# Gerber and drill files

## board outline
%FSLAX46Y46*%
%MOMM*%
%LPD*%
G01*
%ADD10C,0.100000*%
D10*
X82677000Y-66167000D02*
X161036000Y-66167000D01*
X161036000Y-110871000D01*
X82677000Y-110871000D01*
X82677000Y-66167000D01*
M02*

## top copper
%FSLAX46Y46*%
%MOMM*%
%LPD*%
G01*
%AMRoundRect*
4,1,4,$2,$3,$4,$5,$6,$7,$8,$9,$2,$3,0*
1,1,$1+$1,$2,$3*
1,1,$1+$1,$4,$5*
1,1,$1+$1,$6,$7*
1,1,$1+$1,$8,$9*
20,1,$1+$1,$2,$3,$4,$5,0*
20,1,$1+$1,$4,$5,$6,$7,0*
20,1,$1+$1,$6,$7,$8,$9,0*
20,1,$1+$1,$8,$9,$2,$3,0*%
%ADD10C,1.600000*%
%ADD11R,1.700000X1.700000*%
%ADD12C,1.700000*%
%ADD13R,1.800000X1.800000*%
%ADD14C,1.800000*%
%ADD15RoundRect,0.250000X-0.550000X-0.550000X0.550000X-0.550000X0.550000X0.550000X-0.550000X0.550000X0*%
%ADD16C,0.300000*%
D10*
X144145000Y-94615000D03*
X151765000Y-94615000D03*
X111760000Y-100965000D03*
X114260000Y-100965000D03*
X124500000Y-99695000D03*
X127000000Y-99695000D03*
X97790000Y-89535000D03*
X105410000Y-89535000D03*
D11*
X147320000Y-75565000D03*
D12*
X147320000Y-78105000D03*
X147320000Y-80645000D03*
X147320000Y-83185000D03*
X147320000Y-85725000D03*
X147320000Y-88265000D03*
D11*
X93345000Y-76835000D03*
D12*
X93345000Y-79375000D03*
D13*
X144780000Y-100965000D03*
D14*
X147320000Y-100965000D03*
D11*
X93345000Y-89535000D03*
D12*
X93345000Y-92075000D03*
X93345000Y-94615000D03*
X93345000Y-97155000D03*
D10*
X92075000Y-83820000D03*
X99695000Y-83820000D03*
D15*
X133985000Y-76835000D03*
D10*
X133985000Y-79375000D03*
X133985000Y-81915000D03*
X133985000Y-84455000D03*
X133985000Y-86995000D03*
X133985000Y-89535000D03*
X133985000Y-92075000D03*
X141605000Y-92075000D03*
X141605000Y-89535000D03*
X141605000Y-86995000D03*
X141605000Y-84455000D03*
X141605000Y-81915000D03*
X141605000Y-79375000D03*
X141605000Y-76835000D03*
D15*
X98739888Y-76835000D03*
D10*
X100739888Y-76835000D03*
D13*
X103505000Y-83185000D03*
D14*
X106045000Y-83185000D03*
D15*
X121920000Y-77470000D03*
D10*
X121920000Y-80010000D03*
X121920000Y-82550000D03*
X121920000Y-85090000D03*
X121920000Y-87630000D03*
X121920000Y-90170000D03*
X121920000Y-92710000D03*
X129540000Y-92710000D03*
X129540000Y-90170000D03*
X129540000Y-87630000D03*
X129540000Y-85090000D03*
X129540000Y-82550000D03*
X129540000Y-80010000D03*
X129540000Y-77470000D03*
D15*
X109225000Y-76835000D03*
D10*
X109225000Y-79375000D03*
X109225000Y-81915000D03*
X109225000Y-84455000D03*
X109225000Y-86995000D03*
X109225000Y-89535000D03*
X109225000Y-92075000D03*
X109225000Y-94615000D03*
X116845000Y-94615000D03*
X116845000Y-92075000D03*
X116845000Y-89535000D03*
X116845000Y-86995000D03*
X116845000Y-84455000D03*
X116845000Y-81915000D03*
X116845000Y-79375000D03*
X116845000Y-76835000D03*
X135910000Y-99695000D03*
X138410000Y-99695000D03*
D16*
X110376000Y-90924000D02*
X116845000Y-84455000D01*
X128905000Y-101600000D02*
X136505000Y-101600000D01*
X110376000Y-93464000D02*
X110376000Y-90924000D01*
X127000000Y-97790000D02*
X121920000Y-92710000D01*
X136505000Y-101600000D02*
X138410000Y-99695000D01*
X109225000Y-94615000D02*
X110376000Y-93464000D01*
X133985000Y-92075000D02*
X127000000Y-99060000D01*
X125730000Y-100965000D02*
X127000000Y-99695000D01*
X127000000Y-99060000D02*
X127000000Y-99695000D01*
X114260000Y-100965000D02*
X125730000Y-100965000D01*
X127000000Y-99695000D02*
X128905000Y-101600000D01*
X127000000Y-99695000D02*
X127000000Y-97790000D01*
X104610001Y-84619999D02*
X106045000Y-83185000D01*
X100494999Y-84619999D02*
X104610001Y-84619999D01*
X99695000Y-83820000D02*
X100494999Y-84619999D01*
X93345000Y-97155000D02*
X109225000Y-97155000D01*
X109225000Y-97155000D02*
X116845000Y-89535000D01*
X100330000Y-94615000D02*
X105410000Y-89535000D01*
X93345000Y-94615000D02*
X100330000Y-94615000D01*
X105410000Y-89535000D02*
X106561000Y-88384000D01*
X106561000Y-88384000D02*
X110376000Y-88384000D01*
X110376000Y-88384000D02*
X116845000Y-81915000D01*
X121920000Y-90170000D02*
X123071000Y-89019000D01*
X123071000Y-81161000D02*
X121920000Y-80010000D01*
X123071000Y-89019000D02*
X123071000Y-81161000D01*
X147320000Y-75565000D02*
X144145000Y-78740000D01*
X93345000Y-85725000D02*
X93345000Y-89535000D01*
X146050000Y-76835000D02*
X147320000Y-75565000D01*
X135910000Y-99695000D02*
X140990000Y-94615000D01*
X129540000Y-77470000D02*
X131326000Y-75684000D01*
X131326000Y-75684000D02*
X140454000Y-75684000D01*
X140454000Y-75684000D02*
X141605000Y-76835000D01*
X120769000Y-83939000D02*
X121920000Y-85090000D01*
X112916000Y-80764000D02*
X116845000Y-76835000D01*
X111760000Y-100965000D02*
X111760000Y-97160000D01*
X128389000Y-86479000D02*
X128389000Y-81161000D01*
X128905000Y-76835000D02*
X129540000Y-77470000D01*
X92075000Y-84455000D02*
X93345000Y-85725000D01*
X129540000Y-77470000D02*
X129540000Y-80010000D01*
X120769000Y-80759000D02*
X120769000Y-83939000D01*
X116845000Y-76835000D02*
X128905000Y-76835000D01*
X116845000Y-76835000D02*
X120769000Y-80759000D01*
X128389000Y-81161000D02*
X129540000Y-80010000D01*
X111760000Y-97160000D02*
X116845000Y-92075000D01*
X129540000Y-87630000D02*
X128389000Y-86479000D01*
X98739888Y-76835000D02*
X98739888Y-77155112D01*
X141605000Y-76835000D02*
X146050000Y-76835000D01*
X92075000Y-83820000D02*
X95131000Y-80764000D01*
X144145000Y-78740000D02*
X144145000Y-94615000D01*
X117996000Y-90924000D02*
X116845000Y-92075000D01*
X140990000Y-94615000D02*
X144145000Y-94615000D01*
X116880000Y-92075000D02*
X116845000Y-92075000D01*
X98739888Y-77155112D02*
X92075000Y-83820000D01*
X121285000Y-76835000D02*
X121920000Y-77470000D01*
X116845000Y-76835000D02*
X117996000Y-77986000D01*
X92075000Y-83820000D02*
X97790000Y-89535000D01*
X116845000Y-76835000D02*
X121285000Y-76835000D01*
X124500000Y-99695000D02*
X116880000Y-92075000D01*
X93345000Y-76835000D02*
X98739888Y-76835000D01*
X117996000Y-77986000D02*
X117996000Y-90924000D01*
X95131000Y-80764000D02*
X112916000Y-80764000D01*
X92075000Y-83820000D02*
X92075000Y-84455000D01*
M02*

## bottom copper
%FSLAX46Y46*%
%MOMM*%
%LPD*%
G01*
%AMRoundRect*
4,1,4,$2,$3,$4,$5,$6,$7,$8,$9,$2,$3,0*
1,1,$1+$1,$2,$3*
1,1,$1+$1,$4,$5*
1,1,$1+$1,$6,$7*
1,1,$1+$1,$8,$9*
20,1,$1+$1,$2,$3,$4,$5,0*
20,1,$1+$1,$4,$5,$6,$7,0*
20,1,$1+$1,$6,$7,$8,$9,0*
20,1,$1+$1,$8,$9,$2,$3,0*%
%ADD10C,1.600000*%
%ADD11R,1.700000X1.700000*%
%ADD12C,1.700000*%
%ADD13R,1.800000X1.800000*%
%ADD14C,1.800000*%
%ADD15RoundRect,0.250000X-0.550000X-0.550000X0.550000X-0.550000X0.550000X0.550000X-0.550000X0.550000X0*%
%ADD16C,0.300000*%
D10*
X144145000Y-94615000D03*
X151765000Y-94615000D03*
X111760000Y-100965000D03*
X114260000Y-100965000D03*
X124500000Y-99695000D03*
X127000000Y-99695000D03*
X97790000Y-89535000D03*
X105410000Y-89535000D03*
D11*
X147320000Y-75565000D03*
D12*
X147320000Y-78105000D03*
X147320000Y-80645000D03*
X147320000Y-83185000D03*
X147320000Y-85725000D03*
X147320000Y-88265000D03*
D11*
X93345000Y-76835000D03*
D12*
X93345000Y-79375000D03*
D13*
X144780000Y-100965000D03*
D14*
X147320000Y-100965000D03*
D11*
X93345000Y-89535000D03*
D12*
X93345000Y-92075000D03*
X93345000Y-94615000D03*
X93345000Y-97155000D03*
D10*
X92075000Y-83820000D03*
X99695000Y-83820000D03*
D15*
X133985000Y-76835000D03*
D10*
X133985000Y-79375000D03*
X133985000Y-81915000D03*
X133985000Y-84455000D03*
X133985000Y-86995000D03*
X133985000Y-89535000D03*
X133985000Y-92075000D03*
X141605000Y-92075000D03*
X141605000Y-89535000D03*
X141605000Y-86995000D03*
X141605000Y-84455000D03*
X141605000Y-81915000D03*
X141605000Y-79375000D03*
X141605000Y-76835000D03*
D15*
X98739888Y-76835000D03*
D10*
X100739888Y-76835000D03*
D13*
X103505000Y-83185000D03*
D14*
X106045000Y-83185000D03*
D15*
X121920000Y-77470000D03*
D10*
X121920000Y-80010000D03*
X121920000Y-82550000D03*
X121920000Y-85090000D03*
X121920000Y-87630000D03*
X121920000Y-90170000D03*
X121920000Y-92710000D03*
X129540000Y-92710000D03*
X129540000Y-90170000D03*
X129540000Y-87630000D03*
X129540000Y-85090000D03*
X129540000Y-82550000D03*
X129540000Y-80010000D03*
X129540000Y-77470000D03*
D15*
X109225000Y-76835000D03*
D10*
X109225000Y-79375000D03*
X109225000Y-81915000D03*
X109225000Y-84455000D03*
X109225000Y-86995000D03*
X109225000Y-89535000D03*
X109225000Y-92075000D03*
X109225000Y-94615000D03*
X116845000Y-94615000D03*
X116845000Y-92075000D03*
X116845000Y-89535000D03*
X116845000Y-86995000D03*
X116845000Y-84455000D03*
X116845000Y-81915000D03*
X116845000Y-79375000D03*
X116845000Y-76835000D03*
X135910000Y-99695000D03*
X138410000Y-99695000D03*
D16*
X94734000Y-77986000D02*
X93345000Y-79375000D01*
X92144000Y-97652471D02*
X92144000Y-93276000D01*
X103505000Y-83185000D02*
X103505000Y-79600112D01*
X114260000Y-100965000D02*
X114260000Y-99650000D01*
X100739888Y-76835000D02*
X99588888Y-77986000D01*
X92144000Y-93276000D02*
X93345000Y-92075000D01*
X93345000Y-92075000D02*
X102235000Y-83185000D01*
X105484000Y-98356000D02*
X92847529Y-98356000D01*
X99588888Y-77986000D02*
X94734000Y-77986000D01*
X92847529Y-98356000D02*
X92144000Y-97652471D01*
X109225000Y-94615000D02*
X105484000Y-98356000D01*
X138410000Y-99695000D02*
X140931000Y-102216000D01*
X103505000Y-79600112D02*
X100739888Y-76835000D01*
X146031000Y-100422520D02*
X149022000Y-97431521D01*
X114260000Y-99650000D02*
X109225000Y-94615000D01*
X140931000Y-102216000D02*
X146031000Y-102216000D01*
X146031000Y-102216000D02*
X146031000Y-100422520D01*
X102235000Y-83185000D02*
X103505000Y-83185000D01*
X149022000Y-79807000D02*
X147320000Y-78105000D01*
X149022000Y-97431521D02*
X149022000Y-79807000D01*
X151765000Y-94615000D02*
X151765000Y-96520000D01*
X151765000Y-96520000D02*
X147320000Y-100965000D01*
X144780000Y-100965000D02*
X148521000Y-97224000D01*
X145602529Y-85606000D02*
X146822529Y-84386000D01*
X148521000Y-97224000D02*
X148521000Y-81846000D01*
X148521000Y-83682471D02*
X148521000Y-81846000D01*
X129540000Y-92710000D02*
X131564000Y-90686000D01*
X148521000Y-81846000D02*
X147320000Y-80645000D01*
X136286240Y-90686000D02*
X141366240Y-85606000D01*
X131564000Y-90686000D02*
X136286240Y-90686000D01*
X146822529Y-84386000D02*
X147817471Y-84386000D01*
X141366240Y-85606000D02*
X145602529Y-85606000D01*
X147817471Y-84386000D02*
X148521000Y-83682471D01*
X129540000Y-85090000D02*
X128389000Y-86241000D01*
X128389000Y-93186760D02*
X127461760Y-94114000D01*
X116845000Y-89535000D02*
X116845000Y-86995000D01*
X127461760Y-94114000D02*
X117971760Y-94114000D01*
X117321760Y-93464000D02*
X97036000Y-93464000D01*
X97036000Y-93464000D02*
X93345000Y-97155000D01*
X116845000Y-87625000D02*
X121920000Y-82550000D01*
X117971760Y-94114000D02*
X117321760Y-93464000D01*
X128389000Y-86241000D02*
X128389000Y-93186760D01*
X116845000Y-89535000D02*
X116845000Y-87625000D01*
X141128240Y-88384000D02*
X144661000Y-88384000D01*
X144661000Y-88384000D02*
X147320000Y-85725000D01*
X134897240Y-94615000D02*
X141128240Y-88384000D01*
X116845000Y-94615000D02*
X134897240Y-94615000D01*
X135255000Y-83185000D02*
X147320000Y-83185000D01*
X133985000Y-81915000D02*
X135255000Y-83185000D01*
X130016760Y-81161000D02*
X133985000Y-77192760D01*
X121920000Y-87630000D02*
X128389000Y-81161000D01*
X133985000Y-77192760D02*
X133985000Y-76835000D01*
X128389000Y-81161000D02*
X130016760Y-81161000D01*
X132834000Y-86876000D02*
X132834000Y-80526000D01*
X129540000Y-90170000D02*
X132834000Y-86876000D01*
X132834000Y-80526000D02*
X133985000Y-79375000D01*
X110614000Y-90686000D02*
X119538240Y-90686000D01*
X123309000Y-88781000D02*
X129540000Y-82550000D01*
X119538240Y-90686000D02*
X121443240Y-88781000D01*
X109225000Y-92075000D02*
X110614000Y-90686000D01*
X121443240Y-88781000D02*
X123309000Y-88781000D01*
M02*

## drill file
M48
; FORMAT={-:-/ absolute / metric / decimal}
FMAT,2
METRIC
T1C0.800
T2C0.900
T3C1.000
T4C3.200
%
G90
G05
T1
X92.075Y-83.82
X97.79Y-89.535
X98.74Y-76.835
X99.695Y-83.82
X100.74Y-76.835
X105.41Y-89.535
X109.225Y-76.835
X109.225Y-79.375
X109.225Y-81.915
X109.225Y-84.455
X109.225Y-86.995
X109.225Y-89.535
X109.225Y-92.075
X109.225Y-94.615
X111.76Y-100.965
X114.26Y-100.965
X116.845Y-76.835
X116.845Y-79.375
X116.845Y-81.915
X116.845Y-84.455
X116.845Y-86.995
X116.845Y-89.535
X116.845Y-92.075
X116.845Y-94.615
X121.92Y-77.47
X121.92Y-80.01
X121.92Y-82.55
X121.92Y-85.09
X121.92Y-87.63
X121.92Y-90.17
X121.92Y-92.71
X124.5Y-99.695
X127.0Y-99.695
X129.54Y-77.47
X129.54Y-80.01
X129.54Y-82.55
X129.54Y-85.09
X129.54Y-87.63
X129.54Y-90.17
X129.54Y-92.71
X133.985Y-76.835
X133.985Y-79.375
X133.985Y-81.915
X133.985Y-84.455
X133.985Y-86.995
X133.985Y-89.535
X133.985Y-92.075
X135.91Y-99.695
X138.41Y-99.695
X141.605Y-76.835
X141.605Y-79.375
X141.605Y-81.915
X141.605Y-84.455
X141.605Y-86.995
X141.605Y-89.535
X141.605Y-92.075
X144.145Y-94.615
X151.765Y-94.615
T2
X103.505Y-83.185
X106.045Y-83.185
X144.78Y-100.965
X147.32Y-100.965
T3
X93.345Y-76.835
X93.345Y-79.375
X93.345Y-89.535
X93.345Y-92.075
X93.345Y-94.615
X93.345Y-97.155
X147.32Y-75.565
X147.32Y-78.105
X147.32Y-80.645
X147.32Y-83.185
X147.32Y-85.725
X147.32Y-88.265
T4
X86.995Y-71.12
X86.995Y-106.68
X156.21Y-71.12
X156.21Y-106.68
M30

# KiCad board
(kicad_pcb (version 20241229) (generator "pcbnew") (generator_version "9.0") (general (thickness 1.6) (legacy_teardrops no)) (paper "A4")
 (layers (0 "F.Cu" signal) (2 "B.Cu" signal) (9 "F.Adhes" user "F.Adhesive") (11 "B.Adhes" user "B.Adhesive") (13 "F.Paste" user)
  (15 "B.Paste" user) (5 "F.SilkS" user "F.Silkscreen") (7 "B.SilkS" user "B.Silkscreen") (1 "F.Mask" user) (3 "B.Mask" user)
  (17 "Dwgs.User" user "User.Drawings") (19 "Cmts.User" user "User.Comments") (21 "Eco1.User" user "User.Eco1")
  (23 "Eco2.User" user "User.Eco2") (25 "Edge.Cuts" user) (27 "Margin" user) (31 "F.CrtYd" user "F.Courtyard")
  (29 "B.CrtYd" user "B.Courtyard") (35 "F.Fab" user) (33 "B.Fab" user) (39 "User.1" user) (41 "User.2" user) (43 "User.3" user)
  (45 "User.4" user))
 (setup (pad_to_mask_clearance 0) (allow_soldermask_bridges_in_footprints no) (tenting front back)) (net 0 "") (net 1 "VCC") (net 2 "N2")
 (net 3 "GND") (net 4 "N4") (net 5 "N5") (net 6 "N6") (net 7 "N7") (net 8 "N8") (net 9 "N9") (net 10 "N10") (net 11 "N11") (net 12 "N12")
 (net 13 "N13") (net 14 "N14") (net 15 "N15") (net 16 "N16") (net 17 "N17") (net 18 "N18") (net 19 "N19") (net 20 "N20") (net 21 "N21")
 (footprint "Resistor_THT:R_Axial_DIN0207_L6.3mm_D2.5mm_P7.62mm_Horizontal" (layer "F.Cu") (at 144.145 94.615)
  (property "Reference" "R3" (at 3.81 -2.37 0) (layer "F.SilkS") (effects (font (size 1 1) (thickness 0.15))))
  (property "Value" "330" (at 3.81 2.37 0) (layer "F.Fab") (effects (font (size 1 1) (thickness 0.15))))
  (pad "1" thru_hole circle (at 0 0) (size 1.6 1.6) (drill 0.8) (layers "*.Cu" "*.Mask") (remove_unused_layers no) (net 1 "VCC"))
  (pad "2" thru_hole circle (at 7.62 0) (size 1.6 1.6) (drill 0.8) (layers "*.Cu" "*.Mask") (remove_unused_layers no) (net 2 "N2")))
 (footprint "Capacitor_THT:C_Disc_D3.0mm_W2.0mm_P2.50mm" (layer "F.Cu") (at 111.76 100.965)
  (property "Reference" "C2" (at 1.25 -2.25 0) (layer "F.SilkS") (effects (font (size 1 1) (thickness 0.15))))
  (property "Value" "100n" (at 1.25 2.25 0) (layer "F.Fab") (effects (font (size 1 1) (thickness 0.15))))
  (pad "1" thru_hole circle (at 0 0) (size 1.6 1.6) (drill 0.8) (layers "*.Cu" "*.Mask") (remove_unused_layers no) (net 1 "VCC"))
  (pad "2" thru_hole circle (at 2.5 0) (size 1.6 1.6) (drill 0.8) (layers "*.Cu" "*.Mask") (remove_unused_layers no) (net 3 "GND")))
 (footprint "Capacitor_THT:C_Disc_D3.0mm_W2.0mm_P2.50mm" (layer "F.Cu") (at 124.5 99.695)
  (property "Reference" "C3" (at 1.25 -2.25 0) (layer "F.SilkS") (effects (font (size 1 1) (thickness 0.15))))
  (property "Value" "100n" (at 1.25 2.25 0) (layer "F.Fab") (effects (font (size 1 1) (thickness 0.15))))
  (pad "1" thru_hole circle (at 0 0) (size 1.6 1.6) (drill 0.8) (layers "*.Cu" "*.Mask") (remove_unused_layers no) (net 1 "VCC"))
  (pad "2" thru_hole circle (at 2.5 0) (size 1.6 1.6) (drill 0.8) (layers "*.Cu" "*.Mask") (remove_unused_layers no) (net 3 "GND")))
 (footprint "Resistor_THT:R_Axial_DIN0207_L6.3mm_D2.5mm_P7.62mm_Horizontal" (layer "F.Cu") (at 97.79 89.535)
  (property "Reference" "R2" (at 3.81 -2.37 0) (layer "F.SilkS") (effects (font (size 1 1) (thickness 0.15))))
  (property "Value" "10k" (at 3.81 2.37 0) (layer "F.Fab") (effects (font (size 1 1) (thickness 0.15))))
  (pad "1" thru_hole circle (at 0 0) (size 1.6 1.6) (drill 0.8) (layers "*.Cu" "*.Mask") (remove_unused_layers no) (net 1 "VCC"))
  (pad "2" thru_hole circle (at 7.62 0) (size 1.6 1.6) (drill 0.8) (layers "*.Cu" "*.Mask") (remove_unused_layers no) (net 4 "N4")))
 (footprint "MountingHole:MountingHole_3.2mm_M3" (layer "F.Cu") (at 86.995 71.12)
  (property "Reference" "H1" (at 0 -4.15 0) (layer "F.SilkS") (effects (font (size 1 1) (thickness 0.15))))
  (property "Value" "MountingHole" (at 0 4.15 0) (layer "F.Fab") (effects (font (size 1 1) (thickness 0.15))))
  (pad "" np_thru_hole circle (at 0 0) (size 3.2 3.2) (drill 3.2) (layers "*.Cu" "*.Mask")))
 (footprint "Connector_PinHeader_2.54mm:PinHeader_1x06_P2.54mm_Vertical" (layer "F.Cu") (at 147.32 75.565)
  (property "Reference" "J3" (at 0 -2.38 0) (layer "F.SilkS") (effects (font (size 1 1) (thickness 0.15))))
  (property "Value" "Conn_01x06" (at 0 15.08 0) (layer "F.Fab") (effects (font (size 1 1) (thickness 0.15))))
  (pad "1" thru_hole rect (at 0 0) (size 1.7 1.7) (drill 1) (layers "*.Cu" "*.Mask") (remove_unused_layers no) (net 1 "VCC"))
  (pad "2" thru_hole circle (at 0 2.54) (size 1.7 1.7) (drill 1) (layers "*.Cu" "*.Mask") (remove_unused_layers no) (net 3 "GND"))
  (pad "3" thru_hole circle (at 0 5.08) (size 1.7 1.7) (drill 1) (layers "*.Cu" "*.Mask") (remove_unused_layers no) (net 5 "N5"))
  (pad "4" thru_hole circle (at 0 7.62) (size 1.7 1.7) (drill 1) (layers "*.Cu" "*.Mask") (remove_unused_layers no) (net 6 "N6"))
  (pad "5" thru_hole circle (at 0 10.16) (size 1.7 1.7) (drill 1) (layers "*.Cu" "*.Mask") (remove_unused_layers no) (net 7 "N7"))
  (pad "6" thru_hole circle (at 0 12.7) (size 1.7 1.7) (drill 1) (layers "*.Cu" "*.Mask") (remove_unused_layers no) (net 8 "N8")))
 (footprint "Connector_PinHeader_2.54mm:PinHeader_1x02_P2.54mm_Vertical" (layer "F.Cu") (at 93.345 76.835)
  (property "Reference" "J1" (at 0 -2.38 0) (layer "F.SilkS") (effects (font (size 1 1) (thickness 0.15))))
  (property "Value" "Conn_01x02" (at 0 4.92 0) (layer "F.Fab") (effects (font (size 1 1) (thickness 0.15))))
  (pad "1" thru_hole rect (at 0 0) (size 1.7 1.7) (drill 1) (layers "*.Cu" "*.Mask") (remove_unused_layers no) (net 1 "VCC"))
  (pad "2" thru_hole circle (at 0 2.54) (size 1.7 1.7) (drill 1) (layers "*.Cu" "*.Mask") (remove_unused_layers no) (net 3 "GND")))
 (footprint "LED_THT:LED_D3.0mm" (layer "F.Cu") (at 144.78 100.965)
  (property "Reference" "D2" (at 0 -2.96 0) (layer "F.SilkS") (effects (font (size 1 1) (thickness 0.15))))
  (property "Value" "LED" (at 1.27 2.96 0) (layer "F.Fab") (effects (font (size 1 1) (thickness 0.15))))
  (pad "1" thru_hole rect (at 0 0) (size 1.8 1.8) (drill 0.9) (layers "*.Cu" "*.Mask") (remove_unused_layers no) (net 5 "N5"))
  (pad "2" thru_hole circle (at 2.54 0) (size 1.8 1.8) (drill 0.9) (layers "*.Cu" "*.Mask") (remove_unused_layers no) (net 2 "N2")))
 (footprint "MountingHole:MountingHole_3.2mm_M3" (layer "F.Cu") (at 86.995 106.68)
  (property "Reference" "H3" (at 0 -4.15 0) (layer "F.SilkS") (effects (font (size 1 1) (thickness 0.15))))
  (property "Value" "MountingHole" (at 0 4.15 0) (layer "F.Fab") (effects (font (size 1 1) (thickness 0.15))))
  (pad "" np_thru_hole circle (at 0 0) (size 3.2 3.2) (drill 3.2) (layers "*.Cu" "*.Mask")))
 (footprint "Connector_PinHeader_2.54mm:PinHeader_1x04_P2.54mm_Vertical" (layer "F.Cu") (at 93.345 89.535)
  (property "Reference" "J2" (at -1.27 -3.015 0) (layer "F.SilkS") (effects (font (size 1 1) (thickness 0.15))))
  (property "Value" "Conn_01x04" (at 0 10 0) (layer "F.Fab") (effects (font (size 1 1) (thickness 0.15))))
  (pad "1" thru_hole rect (at 0 0) (size 1.7 1.7) (drill 1) (layers "*.Cu" "*.Mask") (remove_unused_layers no) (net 1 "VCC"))
  (pad "2" thru_hole circle (at 0 2.54) (size 1.7 1.7) (drill 1) (layers "*.Cu" "*.Mask") (remove_unused_layers no) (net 3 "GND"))
  (pad "3" thru_hole circle (at 0 5.08) (size 1.7 1.7) (drill 1) (layers "*.Cu" "*.Mask") (remove_unused_layers no) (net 4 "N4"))
  (pad "4" thru_hole circle (at 0 7.62) (size 1.7 1.7) (drill 1) (layers "*.Cu" "*.Mask") (remove_unused_layers no) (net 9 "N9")))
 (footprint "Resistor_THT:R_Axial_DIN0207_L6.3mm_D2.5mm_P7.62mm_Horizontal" (layer "F.Cu") (at 92.075 83.82)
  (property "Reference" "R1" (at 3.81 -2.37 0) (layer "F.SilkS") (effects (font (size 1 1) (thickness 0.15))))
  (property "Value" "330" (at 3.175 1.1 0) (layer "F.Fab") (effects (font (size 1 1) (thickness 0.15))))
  (pad "1" thru_hole circle (at 0 0) (size 1.6 1.6) (drill 0.8) (layers "*.Cu" "*.Mask") (remove_unused_layers no) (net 1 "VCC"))
  (pad "2" thru_hole circle (at 7.62 0) (size 1.6 1.6) (drill 0.8) (layers "*.Cu" "*.Mask") (remove_unused_layers no) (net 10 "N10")))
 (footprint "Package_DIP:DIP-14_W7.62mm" (layer "F.Cu") (at 133.985 76.835)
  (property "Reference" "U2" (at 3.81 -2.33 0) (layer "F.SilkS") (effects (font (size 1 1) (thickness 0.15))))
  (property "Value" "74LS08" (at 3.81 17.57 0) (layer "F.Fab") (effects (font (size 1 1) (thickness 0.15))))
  (pad "1" thru_hole roundrect (at 0 0) (size 1.6 1.6) (drill 0.8) (layers "*.Cu" "*.Mask") (remove_unused_layers no)
   (roundrect_rratio 0.15625) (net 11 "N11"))
  (pad "2" thru_hole circle (at 0 2.54) (size 1.6 1.6) (drill 0.8) (layers "*.Cu" "*.Mask") (remove_unused_layers no) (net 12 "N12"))
  (pad "3" thru_hole circle (at 0 5.08) (size 1.6 1.6) (drill 0.8) (layers "*.Cu" "*.Mask") (remove_unused_layers no) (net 6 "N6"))
  (pad "4" thru_hole circle (at 0 7.62) (size 1.6 1.6) (drill 0.8) (layers "*.Cu" "*.Mask") (remove_unused_layers no))
  (pad "5" thru_hole circle (at 0 10.16) (size 1.6 1.6) (drill 0.8) (layers "*.Cu" "*.Mask") (remove_unused_layers no))
  (pad "6" thru_hole circle (at 0 12.7) (size 1.6 1.6) (drill 0.8) (layers "*.Cu" "*.Mask") (remove_unused_layers no))
  (pad "7" thru_hole circle (at 0 15.24) (size 1.6 1.6) (drill 0.8) (layers "*.Cu" "*.Mask") (remove_unused_layers no) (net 3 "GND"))
  (pad "8" thru_hole circle (at 7.62 15.24) (size 1.6 1.6) (drill 0.8) (layers "*.Cu" "*.Mask") (remove_unused_layers no))
  (pad "9" thru_hole circle (at 7.62 12.7) (size 1.6 1.6) (drill 0.8) (layers "*.Cu" "*.Mask") (remove_unused_layers no))
  (pad "10" thru_hole circle (at 7.62 10.16) (size 1.6 1.6) (drill 0.8) (layers "*.Cu" "*.Mask") (remove_unused_layers no))
  (pad "11" thru_hole circle (at 7.62 7.62) (size 1.6 1.6) (drill 0.8) (layers "*.Cu" "*.Mask") (remove_unused_layers no))
  (pad "12" thru_hole circle (at 7.62 5.08) (size 1.6 1.6) (drill 0.8) (layers "*.Cu" "*.Mask") (remove_unused_layers no))
  (pad "13" thru_hole circle (at 7.62 2.54) (size 1.6 1.6) (drill 0.8) (layers "*.Cu" "*.Mask") (remove_unused_layers no))
  (pad "14" thru_hole circle (at 7.62 0) (size 1.6 1.6) (drill 0.8) (layers "*.Cu" "*.Mask") (remove_unused_layers no) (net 1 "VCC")))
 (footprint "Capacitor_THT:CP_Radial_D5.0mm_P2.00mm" (layer "F.Cu") (at 98.739888 76.835)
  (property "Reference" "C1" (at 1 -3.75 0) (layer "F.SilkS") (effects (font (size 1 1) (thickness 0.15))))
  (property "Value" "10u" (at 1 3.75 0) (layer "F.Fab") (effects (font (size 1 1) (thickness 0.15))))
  (pad "1" thru_hole roundrect (at 0 0) (size 1.6 1.6) (drill 0.8) (layers "*.Cu" "*.Mask") (remove_unused_layers no)
   (roundrect_rratio 0.15625) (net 1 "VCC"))
  (pad "2" thru_hole circle (at 2 0) (size 1.6 1.6) (drill 0.8) (layers "*.Cu" "*.Mask") (remove_unused_layers no) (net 3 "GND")))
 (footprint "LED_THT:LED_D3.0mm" (layer "F.Cu") (at 103.505 83.185)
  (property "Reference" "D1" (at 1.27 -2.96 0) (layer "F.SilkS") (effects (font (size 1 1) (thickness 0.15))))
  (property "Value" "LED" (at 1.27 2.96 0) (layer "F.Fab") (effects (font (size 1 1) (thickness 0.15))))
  (pad "1" thru_hole rect (at 0 0) (size 1.8 1.8) (drill 0.9) (layers "*.Cu" "*.Mask") (remove_unused_layers no) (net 3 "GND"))
  (pad "2" thru_hole circle (at 2.54 0) (size 1.8 1.8) (drill 0.9) (layers "*.Cu" "*.Mask") (remove_unused_layers no) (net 10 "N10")))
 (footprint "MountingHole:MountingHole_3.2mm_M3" (layer "F.Cu") (at 156.21 71.12)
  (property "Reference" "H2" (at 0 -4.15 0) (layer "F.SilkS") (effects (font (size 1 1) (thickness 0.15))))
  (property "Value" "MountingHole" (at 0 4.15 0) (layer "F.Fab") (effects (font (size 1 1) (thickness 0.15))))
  (pad "" np_thru_hole circle (at 0 0) (size 3.2 3.2) (drill 3.2) (layers "*.Cu" "*.Mask")))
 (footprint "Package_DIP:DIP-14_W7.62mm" (layer "F.Cu") (at 121.92 77.47)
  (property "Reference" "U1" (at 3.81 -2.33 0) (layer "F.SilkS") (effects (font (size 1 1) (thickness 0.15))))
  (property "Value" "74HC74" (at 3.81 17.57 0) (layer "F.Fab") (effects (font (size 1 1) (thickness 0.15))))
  (pad "1" thru_hole roundrect (at 0 0) (size 1.6 1.6) (drill 0.8) (layers "*.Cu" "*.Mask") (remove_unused_layers no)
   (roundrect_rratio 0.15625) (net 1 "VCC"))
  (pad "2" thru_hole circle (at 0 2.54) (size 1.6 1.6) (drill 0.8) (layers "*.Cu" "*.Mask") (remove_unused_layers no) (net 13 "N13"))
  (pad "3" thru_hole circle (at 0 5.08) (size 1.6 1.6) (drill 0.8) (layers "*.Cu" "*.Mask") (remove_unused_layers no) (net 9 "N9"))
  (pad "4" thru_hole circle (at 0 7.62) (size 1.6 1.6) (drill 0.8) (layers "*.Cu" "*.Mask") (remove_unused_layers no) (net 1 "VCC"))
  (pad "5" thru_hole circle (at 0 10.16) (size 1.6 1.6) (drill 0.8) (layers "*.Cu" "*.Mask") (remove_unused_layers no) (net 11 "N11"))
  (pad "6" thru_hole circle (at 0 12.7) (size 1.6 1.6) (drill 0.8) (layers "*.Cu" "*.Mask") (remove_unused_layers no) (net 13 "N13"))
  (pad "7" thru_hole circle (at 0 15.24) (size 1.6 1.6) (drill 0.8) (layers "*.Cu" "*.Mask") (remove_unused_layers no) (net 3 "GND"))
  (pad "8" thru_hole circle (at 7.62 15.24) (size 1.6 1.6) (drill 0.8) (layers "*.Cu" "*.Mask") (remove_unused_layers no) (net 5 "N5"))
  (pad "9" thru_hole circle (at 7.62 12.7) (size 1.6 1.6) (drill 0.8) (layers "*.Cu" "*.Mask") (remove_unused_layers no) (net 12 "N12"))
  (pad "10" thru_hole circle (at 7.62 10.16) (size 1.6 1.6) (drill 0.8) (layers "*.Cu" "*.Mask") (remove_unused_layers no) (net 1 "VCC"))
  (pad "11" thru_hole circle (at 7.62 7.62) (size 1.6 1.6) (drill 0.8) (layers "*.Cu" "*.Mask") (remove_unused_layers no) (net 9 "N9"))
  (pad "12" thru_hole circle (at 7.62 5.08) (size 1.6 1.6) (drill 0.8) (layers "*.Cu" "*.Mask") (remove_unused_layers no) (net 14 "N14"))
  (pad "13" thru_hole circle (at 7.62 2.54) (size 1.6 1.6) (drill 0.8) (layers "*.Cu" "*.Mask") (remove_unused_layers no) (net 1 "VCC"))
  (pad "14" thru_hole circle (at 7.62 0) (size 1.6 1.6) (drill 0.8) (layers "*.Cu" "*.Mask") (remove_unused_layers no) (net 1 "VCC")))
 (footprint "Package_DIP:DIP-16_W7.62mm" (layer "F.Cu") (at 109.225 76.835)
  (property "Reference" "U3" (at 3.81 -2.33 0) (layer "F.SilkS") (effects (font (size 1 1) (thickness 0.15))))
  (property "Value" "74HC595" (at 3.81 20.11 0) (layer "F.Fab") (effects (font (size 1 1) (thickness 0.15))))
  (pad "1" thru_hole roundrect (at 0 0) (size 1.6 1.6) (drill 0.8) (layers "*.Cu" "*.Mask") (remove_unused_layers no)
   (roundrect_rratio 0.15625) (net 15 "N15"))
  (pad "2" thru_hole circle (at 0 2.54) (size 1.6 1.6) (drill 0.8) (layers "*.Cu" "*.Mask") (remove_unused_layers no) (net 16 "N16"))
  (pad "3" thru_hole circle (at 0 5.08) (size 1.6 1.6) (drill 0.8) (layers "*.Cu" "*.Mask") (remove_unused_layers no) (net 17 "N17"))
  (pad "4" thru_hole circle (at 0 7.62) (size 1.6 1.6) (drill 0.8) (layers "*.Cu" "*.Mask") (remove_unused_layers no) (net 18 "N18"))
  (pad "5" thru_hole circle (at 0 10.16) (size 1.6 1.6) (drill 0.8) (layers "*.Cu" "*.Mask") (remove_unused_layers no) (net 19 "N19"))
  (pad "6" thru_hole circle (at 0 12.7) (size 1.6 1.6) (drill 0.8) (layers "*.Cu" "*.Mask") (remove_unused_layers no) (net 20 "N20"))
  (pad "7" thru_hole circle (at 0 15.24) (size 1.6 1.6) (drill 0.8) (layers "*.Cu" "*.Mask") (remove_unused_layers no) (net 14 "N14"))
  (pad "8" thru_hole circle (at 0 17.78) (size 1.6 1.6) (drill 0.8) (layers "*.Cu" "*.Mask") (remove_unused_layers no) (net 3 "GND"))
  (pad "9" thru_hole circle (at 7.62 17.78) (size 1.6 1.6) (drill 0.8) (layers "*.Cu" "*.Mask") (remove_unused_layers no) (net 7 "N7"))
  (pad "10" thru_hole circle (at 7.62 15.24) (size 1.6 1.6) (drill 0.8) (layers "*.Cu" "*.Mask") (remove_unused_layers no) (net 1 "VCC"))
  (pad "11" thru_hole circle (at 7.62 12.7) (size 1.6 1.6) (drill 0.8) (layers "*.Cu" "*.Mask") (remove_unused_layers no) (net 9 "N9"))
  (pad "12" thru_hole circle (at 7.62 10.16) (size 1.6 1.6) (drill 0.8) (layers "*.Cu" "*.Mask") (remove_unused_layers no) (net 9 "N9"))
  (pad "13" thru_hole circle (at 7.62 7.62) (size 1.6 1.6) (drill 0.8) (layers "*.Cu" "*.Mask") (remove_unused_layers no) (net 3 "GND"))
  (pad "14" thru_hole circle (at 7.62 5.08) (size 1.6 1.6) (drill 0.8) (layers "*.Cu" "*.Mask") (remove_unused_layers no) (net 4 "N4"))
  (pad "15" thru_hole circle (at 7.62 2.54) (size 1.6 1.6) (drill 0.8) (layers "*.Cu" "*.Mask") (remove_unused_layers no) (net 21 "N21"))
  (pad "16" thru_hole circle (at 7.62 0) (size 1.6 1.6) (drill 0.8) (layers "*.Cu" "*.Mask") (remove_unused_layers no) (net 1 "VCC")))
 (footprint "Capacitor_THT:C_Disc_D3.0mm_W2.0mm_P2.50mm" (layer "F.Cu") (at 135.91 99.695)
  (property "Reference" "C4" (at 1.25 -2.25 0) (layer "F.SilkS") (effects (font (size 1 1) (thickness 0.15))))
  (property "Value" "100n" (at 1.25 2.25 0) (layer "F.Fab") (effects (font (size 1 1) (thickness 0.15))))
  (pad "1" thru_hole circle (at 0 0) (size 1.6 1.6) (drill 0.8) (layers "*.Cu" "*.Mask") (remove_unused_layers no) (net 1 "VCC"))
  (pad "2" thru_hole circle (at 2.5 0) (size 1.6 1.6) (drill 0.8) (layers "*.Cu" "*.Mask") (remove_unused_layers no) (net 3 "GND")))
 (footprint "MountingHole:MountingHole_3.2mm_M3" (layer "F.Cu") (at 156.21 106.68)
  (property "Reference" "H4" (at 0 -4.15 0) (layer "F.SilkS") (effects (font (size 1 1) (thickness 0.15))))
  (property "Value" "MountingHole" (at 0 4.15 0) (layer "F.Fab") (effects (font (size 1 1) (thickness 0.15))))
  (pad "" np_thru_hole circle (at 0 0) (size 3.2 3.2) (drill 3.2) (layers "*.Cu" "*.Mask")))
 (gr_rect (start 82.677 66.167) (end 161.036 110.871) (stroke (width 0.1) (type default)) (fill no) (layer "Edge.Cuts"))
 (segment (start 110.376 90.924) (end 116.845 84.455) (width 0.3) (layer "F.Cu") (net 3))
 (segment (start 128.905 101.6) (end 136.505 101.6) (width 0.3) (layer "F.Cu") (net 3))
 (segment (start 110.376 93.464) (end 110.376 90.924) (width 0.3) (layer "F.Cu") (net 3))
 (segment (start 127 97.79) (end 121.92 92.71) (width 0.3) (layer "F.Cu") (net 3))
 (segment (start 136.505 101.6) (end 138.41 99.695) (width 0.3) (layer "F.Cu") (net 3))
 (segment (start 109.225 94.615) (end 110.376 93.464) (width 0.3) (layer "F.Cu") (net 3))
 (segment (start 133.985 92.075) (end 127 99.06) (width 0.3) (layer "F.Cu") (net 3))
 (segment (start 125.73 100.965) (end 127 99.695) (width 0.3) (layer "F.Cu") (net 3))
 (segment (start 127 99.06) (end 127 99.695) (width 0.3) (layer "F.Cu") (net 3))
 (segment (start 114.26 100.965) (end 125.73 100.965) (width 0.3) (layer "F.Cu") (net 3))
 (segment (start 127 99.695) (end 128.905 101.6) (width 0.3) (layer "F.Cu") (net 3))
 (segment (start 127 99.695) (end 127 97.79) (width 0.3) (layer "F.Cu") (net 3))
 (segment (start 94.734 77.986) (end 93.345 79.375) (width 0.3) (layer "B.Cu") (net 3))
 (segment (start 92.144 97.652471) (end 92.144 93.276) (width 0.3) (layer "B.Cu") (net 3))
 (segment (start 103.505 83.185) (end 103.505 79.600112) (width 0.3) (layer "B.Cu") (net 3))
 (segment (start 114.26 100.965) (end 114.26 99.65) (width 0.3) (layer "B.Cu") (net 3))
 (segment (start 100.739888 76.835) (end 99.588888 77.986) (width 0.3) (layer "B.Cu") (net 3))
 (segment (start 92.144 93.276) (end 93.345 92.075) (width 0.3) (layer "B.Cu") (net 3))
 (segment (start 93.345 92.075) (end 102.235 83.185) (width 0.3) (layer "B.Cu") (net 3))
 (segment (start 105.484 98.356) (end 92.847529 98.356) (width 0.3) (layer "B.Cu") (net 3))
 (segment (start 99.588888 77.986) (end 94.734 77.986) (width 0.3) (layer "B.Cu") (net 3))
 (segment (start 92.847529 98.356) (end 92.144 97.652471) (width 0.3) (layer "B.Cu") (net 3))
 (segment (start 109.225 94.615) (end 105.484 98.356) (width 0.3) (layer "B.Cu") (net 3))
 (segment (start 138.41 99.695) (end 140.931 102.216) (width 0.3) (layer "B.Cu") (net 3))
 (segment (start 103.505 79.600112) (end 100.739888 76.835) (width 0.3) (layer "B.Cu") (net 3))
 (segment (start 146.031 100.42252) (end 149.022 97.431521) (width 0.3) (layer "B.Cu") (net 3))
 (segment (start 114.26 99.65) (end 109.225 94.615) (width 0.3) (layer "B.Cu") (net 3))
 (segment (start 140.931 102.216) (end 146.031 102.216) (width 0.3) (layer "B.Cu") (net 3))
 (segment (start 146.031 102.216) (end 146.031 100.42252) (width 0.3) (layer "B.Cu") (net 3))
 (segment (start 102.235 83.185) (end 103.505 83.185) (width 0.3) (layer "B.Cu") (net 3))
 (segment (start 149.022 79.807) (end 147.32 78.105) (width 0.3) (layer "B.Cu") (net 3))
 (segment (start 149.022 97.431521) (end 149.022 79.807) (width 0.3) (layer "B.Cu") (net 3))
 (segment (start 104.610001 84.619999) (end 106.045 83.185) (width 0.3) (layer "F.Cu") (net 10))
 (segment (start 100.494999 84.619999) (end 104.610001 84.619999) (width 0.3) (layer "F.Cu") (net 10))
 (segment (start 99.695 83.82) (end 100.494999 84.619999) (width 0.3) (layer "F.Cu") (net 10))
 (segment (start 151.765 94.615) (end 151.765 96.52) (width 0.3) (layer "B.Cu") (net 2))
 (segment (start 151.765 96.52) (end 147.32 100.965) (width 0.3) (layer "B.Cu") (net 2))
 (segment (start 144.78 100.965) (end 148.521 97.224) (width 0.3) (layer "B.Cu") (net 5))
 (segment (start 145.602529 85.606) (end 146.822529 84.386) (width 0.3) (layer "B.Cu") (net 5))
 (segment (start 148.521 97.224) (end 148.521 81.846) (width 0.3) (layer "B.Cu") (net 5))
 (segment (start 148.521 83.682471) (end 148.521 81.846) (width 0.3) (layer "B.Cu") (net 5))
 (segment (start 129.54 92.71) (end 131.564 90.686) (width 0.3) (layer "B.Cu") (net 5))
 (segment (start 148.521 81.846) (end 147.32 80.645) (width 0.3) (layer "B.Cu") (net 5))
 (segment (start 136.28624 90.686) (end 141.36624 85.606) (width 0.3) (layer "B.Cu") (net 5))
 (segment (start 131.564 90.686) (end 136.28624 90.686) (width 0.3) (layer "B.Cu") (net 5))
 (segment (start 146.822529 84.386) (end 147.817471 84.386) (width 0.3) (layer "B.Cu") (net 5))
 (segment (start 141.36624 85.606) (end 145.602529 85.606) (width 0.3) (layer "B.Cu") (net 5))
 (segment (start 147.817471 84.386) (end 148.521 83.682471) (width 0.3) (layer "B.Cu") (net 5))
 (segment (start 93.345 97.155) (end 109.225 97.155) (width 0.3) (layer "F.Cu") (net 9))
 (segment (start 109.225 97.155) (end 116.845 89.535) (width 0.3) (layer "F.Cu") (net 9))
 (segment (start 129.54 85.09) (end 128.389 86.241) (width 0.3) (layer "B.Cu") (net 9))
 (segment (start 128.389 93.18676) (end 127.46176 94.114) (width 0.3) (layer "B.Cu") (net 9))
 (segment (start 116.845 89.535) (end 116.845 86.995) (width 0.3) (layer "B.Cu") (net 9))
 (segment (start 127.46176 94.114) (end 117.97176 94.114) (width 0.3) (layer "B.Cu") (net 9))
 (segment (start 117.32176 93.464) (end 97.036 93.464) (width 0.3) (layer "B.Cu") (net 9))
 (segment (start 97.036 93.464) (end 93.345 97.155) (width 0.3) (layer "B.Cu") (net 9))
 (segment (start 116.845 87.625) (end 121.92 82.55) (width 0.3) (layer "B.Cu") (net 9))
 (segment (start 117.97176 94.114) (end 117.32176 93.464) (width 0.3) (layer "B.Cu") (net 9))
 (segment (start 128.389 86.241) (end 128.389 93.18676) (width 0.3) (layer "B.Cu") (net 9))
 (segment (start 116.845 89.535) (end 116.845 87.625) (width 0.3) (layer "B.Cu") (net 9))
 (segment (start 100.33 94.615) (end 105.41 89.535) (width 0.3) (layer "F.Cu") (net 4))
 (segment (start 93.345 94.615) (end 100.33 94.615) (width 0.3) (layer "F.Cu") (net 4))
 (segment (start 105.41 89.535) (end 106.561 88.384) (width 0.3) (layer "F.Cu") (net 4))
 (segment (start 106.561 88.384) (end 110.376 88.384) (width 0.3) (layer "F.Cu") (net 4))
 (segment (start 110.376 88.384) (end 116.845 81.915) (width 0.3) (layer "F.Cu") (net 4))
 (segment (start 141.12824 88.384) (end 144.661 88.384) (width 0.3) (layer "B.Cu") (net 7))
 (segment (start 144.661 88.384) (end 147.32 85.725) (width 0.3) (layer "B.Cu") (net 7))
 (segment (start 134.89724 94.615) (end 141.12824 88.384) (width 0.3) (layer "B.Cu") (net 7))
 (segment (start 116.845 94.615) (end 134.89724 94.615) (width 0.3) (layer "B.Cu") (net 7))
 (segment (start 135.255 83.185) (end 147.32 83.185) (width 0.3) (layer "B.Cu") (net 6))
 (segment (start 133.985 81.915) (end 135.255 83.185) (width 0.3) (layer "B.Cu") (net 6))
 (segment (start 130.01676 81.161) (end 133.985 77.19276) (width 0.3) (layer "B.Cu") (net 11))
 (segment (start 121.92 87.63) (end 128.389 81.161) (width 0.3) (layer "B.Cu") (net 11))
 (segment (start 133.985 77.19276) (end 133.985 76.835) (width 0.3) (layer "B.Cu") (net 11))
 (segment (start 128.389 81.161) (end 130.01676 81.161) (width 0.3) (layer "B.Cu") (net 11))
 (segment (start 132.834 86.876) (end 132.834 80.526) (width 0.3) (layer "B.Cu") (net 12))
 (segment (start 129.54 90.17) (end 132.834 86.876) (width 0.3) (layer "B.Cu") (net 12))
 (segment (start 132.834 80.526) (end 133.985 79.375) (width 0.3) (layer "B.Cu") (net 12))
 (segment (start 121.92 90.17) (end 123.071 89.019) (width 0.3) (layer "F.Cu") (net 13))
 (segment (start 123.071 81.161) (end 121.92 80.01) (width 0.3) (layer "F.Cu") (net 13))
 (segment (start 123.071 89.019) (end 123.071 81.161) (width 0.3) (layer "F.Cu") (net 13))
 (segment (start 110.614 90.686) (end 119.53824 90.686) (width 0.3) (layer "B.Cu") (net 14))
 (segment (start 123.309 88.781) (end 129.54 82.55) (width 0.3) (layer "B.Cu") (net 14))
 (segment (start 119.53824 90.686) (end 121.44324 88.781) (width 0.3) (layer "B.Cu") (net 14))
 (segment (start 109.225 92.075) (end 110.614 90.686) (width 0.3) (layer "B.Cu") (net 14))
 (segment (start 121.44324 88.781) (end 123.309 88.781) (width 0.3) (layer "B.Cu") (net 14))
 (segment (start 147.32 75.565) (end 144.145 78.74) (width 0.3) (layer "F.Cu") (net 1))
 (segment (start 93.345 85.725) (end 93.345 89.535) (width 0.3) (layer "F.Cu") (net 1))
 (segment (start 146.05 76.835) (end 147.32 75.565) (width 0.3) (layer "F.Cu") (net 1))
 (segment (start 135.91 99.695) (end 140.99 94.615) (width 0.3) (layer "F.Cu") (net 1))
 (segment (start 129.54 77.47) (end 131.326 75.684) (width 0.3) (layer "F.Cu") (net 1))
 (segment (start 131.326 75.684) (end 140.454 75.684) (width 0.3) (layer "F.Cu") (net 1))
 (segment (start 140.454 75.684) (end 141.605 76.835) (width 0.3) (layer "F.Cu") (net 1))
 (segment (start 120.769 83.939) (end 121.92 85.09) (width 0.3) (layer "F.Cu") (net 1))
 (segment (start 112.916 80.764) (end 116.845 76.835) (width 0.3) (layer "F.Cu") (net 1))
 (segment (start 111.76 100.965) (end 111.76 97.16) (width 0.3) (layer "F.Cu") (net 1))
 (segment (start 128.389 86.479) (end 128.389 81.161) (width 0.3) (layer "F.Cu") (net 1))
 (segment (start 128.905 76.835) (end 129.54 77.47) (width 0.3) (layer "F.Cu") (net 1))
 (segment (start 92.075 84.455) (end 93.345 85.725) (width 0.3) (layer "F.Cu") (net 1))
 (segment (start 129.54 77.47) (end 129.54 80.01) (width 0.3) (layer "F.Cu") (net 1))
 (segment (start 120.769 80.759) (end 120.769 83.939) (width 0.3) (layer "F.Cu") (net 1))
 (segment (start 116.845 76.835) (end 128.905 76.835) (width 0.3) (layer "F.Cu") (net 1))
 (segment (start 116.845 76.835) (end 120.769 80.759) (width 0.3) (layer "F.Cu") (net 1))
 (segment (start 128.389 81.161) (end 129.54 80.01) (width 0.3) (layer "F.Cu") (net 1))
 (segment (start 111.76 97.16) (end 116.845 92.075) (width 0.3) (layer "F.Cu") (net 1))
 (segment (start 129.54 87.63) (end 128.389 86.479) (width 0.3) (layer "F.Cu") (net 1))
 (segment (start 98.739888 76.835) (end 98.739888 77.155112) (width 0.3) (layer "F.Cu") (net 1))
 (segment (start 141.605 76.835) (end 146.05 76.835) (width 0.3) (layer "F.Cu") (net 1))
 (segment (start 92.075 83.82) (end 95.131 80.764) (width 0.3) (layer "F.Cu") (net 1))
 (segment (start 144.145 78.74) (end 144.145 94.615) (width 0.3) (layer "F.Cu") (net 1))
 (segment (start 117.996 90.924) (end 116.845 92.075) (width 0.3) (layer "F.Cu") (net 1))
 (segment (start 140.99 94.615) (end 144.145 94.615) (width 0.3) (layer "F.Cu") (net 1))
 (segment (start 116.88 92.075) (end 116.845 92.075) (width 0.3) (layer "F.Cu") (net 1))
 (segment (start 98.739888 77.155112) (end 92.075 83.82) (width 0.3) (layer "F.Cu") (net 1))
 (segment (start 121.285 76.835) (end 121.92 77.47) (width 0.3) (layer "F.Cu") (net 1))
 (segment (start 116.845 76.835) (end 117.996 77.986) (width 0.3) (layer "F.Cu") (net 1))
 (segment (start 92.075 83.82) (end 97.79 89.535) (width 0.3) (layer "F.Cu") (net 1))
 (segment (start 116.845 76.835) (end 121.285 76.835) (width 0.3) (layer "F.Cu") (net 1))
 (segment (start 124.5 99.695) (end 116.88 92.075) (width 0.3) (layer "F.Cu") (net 1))
 (segment (start 93.345 76.835) (end 98.739888 76.835) (width 0.3) (layer "F.Cu") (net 1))
 (segment (start 117.996 77.986) (end 117.996 90.924) (width 0.3) (layer "F.Cu") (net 1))
 (segment (start 95.131 80.764) (end 112.916 80.764) (width 0.3) (layer "F.Cu") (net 1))
 (segment (start 92.075 83.82) (end 92.075 84.455) (width 0.3) (layer "F.Cu") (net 1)))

